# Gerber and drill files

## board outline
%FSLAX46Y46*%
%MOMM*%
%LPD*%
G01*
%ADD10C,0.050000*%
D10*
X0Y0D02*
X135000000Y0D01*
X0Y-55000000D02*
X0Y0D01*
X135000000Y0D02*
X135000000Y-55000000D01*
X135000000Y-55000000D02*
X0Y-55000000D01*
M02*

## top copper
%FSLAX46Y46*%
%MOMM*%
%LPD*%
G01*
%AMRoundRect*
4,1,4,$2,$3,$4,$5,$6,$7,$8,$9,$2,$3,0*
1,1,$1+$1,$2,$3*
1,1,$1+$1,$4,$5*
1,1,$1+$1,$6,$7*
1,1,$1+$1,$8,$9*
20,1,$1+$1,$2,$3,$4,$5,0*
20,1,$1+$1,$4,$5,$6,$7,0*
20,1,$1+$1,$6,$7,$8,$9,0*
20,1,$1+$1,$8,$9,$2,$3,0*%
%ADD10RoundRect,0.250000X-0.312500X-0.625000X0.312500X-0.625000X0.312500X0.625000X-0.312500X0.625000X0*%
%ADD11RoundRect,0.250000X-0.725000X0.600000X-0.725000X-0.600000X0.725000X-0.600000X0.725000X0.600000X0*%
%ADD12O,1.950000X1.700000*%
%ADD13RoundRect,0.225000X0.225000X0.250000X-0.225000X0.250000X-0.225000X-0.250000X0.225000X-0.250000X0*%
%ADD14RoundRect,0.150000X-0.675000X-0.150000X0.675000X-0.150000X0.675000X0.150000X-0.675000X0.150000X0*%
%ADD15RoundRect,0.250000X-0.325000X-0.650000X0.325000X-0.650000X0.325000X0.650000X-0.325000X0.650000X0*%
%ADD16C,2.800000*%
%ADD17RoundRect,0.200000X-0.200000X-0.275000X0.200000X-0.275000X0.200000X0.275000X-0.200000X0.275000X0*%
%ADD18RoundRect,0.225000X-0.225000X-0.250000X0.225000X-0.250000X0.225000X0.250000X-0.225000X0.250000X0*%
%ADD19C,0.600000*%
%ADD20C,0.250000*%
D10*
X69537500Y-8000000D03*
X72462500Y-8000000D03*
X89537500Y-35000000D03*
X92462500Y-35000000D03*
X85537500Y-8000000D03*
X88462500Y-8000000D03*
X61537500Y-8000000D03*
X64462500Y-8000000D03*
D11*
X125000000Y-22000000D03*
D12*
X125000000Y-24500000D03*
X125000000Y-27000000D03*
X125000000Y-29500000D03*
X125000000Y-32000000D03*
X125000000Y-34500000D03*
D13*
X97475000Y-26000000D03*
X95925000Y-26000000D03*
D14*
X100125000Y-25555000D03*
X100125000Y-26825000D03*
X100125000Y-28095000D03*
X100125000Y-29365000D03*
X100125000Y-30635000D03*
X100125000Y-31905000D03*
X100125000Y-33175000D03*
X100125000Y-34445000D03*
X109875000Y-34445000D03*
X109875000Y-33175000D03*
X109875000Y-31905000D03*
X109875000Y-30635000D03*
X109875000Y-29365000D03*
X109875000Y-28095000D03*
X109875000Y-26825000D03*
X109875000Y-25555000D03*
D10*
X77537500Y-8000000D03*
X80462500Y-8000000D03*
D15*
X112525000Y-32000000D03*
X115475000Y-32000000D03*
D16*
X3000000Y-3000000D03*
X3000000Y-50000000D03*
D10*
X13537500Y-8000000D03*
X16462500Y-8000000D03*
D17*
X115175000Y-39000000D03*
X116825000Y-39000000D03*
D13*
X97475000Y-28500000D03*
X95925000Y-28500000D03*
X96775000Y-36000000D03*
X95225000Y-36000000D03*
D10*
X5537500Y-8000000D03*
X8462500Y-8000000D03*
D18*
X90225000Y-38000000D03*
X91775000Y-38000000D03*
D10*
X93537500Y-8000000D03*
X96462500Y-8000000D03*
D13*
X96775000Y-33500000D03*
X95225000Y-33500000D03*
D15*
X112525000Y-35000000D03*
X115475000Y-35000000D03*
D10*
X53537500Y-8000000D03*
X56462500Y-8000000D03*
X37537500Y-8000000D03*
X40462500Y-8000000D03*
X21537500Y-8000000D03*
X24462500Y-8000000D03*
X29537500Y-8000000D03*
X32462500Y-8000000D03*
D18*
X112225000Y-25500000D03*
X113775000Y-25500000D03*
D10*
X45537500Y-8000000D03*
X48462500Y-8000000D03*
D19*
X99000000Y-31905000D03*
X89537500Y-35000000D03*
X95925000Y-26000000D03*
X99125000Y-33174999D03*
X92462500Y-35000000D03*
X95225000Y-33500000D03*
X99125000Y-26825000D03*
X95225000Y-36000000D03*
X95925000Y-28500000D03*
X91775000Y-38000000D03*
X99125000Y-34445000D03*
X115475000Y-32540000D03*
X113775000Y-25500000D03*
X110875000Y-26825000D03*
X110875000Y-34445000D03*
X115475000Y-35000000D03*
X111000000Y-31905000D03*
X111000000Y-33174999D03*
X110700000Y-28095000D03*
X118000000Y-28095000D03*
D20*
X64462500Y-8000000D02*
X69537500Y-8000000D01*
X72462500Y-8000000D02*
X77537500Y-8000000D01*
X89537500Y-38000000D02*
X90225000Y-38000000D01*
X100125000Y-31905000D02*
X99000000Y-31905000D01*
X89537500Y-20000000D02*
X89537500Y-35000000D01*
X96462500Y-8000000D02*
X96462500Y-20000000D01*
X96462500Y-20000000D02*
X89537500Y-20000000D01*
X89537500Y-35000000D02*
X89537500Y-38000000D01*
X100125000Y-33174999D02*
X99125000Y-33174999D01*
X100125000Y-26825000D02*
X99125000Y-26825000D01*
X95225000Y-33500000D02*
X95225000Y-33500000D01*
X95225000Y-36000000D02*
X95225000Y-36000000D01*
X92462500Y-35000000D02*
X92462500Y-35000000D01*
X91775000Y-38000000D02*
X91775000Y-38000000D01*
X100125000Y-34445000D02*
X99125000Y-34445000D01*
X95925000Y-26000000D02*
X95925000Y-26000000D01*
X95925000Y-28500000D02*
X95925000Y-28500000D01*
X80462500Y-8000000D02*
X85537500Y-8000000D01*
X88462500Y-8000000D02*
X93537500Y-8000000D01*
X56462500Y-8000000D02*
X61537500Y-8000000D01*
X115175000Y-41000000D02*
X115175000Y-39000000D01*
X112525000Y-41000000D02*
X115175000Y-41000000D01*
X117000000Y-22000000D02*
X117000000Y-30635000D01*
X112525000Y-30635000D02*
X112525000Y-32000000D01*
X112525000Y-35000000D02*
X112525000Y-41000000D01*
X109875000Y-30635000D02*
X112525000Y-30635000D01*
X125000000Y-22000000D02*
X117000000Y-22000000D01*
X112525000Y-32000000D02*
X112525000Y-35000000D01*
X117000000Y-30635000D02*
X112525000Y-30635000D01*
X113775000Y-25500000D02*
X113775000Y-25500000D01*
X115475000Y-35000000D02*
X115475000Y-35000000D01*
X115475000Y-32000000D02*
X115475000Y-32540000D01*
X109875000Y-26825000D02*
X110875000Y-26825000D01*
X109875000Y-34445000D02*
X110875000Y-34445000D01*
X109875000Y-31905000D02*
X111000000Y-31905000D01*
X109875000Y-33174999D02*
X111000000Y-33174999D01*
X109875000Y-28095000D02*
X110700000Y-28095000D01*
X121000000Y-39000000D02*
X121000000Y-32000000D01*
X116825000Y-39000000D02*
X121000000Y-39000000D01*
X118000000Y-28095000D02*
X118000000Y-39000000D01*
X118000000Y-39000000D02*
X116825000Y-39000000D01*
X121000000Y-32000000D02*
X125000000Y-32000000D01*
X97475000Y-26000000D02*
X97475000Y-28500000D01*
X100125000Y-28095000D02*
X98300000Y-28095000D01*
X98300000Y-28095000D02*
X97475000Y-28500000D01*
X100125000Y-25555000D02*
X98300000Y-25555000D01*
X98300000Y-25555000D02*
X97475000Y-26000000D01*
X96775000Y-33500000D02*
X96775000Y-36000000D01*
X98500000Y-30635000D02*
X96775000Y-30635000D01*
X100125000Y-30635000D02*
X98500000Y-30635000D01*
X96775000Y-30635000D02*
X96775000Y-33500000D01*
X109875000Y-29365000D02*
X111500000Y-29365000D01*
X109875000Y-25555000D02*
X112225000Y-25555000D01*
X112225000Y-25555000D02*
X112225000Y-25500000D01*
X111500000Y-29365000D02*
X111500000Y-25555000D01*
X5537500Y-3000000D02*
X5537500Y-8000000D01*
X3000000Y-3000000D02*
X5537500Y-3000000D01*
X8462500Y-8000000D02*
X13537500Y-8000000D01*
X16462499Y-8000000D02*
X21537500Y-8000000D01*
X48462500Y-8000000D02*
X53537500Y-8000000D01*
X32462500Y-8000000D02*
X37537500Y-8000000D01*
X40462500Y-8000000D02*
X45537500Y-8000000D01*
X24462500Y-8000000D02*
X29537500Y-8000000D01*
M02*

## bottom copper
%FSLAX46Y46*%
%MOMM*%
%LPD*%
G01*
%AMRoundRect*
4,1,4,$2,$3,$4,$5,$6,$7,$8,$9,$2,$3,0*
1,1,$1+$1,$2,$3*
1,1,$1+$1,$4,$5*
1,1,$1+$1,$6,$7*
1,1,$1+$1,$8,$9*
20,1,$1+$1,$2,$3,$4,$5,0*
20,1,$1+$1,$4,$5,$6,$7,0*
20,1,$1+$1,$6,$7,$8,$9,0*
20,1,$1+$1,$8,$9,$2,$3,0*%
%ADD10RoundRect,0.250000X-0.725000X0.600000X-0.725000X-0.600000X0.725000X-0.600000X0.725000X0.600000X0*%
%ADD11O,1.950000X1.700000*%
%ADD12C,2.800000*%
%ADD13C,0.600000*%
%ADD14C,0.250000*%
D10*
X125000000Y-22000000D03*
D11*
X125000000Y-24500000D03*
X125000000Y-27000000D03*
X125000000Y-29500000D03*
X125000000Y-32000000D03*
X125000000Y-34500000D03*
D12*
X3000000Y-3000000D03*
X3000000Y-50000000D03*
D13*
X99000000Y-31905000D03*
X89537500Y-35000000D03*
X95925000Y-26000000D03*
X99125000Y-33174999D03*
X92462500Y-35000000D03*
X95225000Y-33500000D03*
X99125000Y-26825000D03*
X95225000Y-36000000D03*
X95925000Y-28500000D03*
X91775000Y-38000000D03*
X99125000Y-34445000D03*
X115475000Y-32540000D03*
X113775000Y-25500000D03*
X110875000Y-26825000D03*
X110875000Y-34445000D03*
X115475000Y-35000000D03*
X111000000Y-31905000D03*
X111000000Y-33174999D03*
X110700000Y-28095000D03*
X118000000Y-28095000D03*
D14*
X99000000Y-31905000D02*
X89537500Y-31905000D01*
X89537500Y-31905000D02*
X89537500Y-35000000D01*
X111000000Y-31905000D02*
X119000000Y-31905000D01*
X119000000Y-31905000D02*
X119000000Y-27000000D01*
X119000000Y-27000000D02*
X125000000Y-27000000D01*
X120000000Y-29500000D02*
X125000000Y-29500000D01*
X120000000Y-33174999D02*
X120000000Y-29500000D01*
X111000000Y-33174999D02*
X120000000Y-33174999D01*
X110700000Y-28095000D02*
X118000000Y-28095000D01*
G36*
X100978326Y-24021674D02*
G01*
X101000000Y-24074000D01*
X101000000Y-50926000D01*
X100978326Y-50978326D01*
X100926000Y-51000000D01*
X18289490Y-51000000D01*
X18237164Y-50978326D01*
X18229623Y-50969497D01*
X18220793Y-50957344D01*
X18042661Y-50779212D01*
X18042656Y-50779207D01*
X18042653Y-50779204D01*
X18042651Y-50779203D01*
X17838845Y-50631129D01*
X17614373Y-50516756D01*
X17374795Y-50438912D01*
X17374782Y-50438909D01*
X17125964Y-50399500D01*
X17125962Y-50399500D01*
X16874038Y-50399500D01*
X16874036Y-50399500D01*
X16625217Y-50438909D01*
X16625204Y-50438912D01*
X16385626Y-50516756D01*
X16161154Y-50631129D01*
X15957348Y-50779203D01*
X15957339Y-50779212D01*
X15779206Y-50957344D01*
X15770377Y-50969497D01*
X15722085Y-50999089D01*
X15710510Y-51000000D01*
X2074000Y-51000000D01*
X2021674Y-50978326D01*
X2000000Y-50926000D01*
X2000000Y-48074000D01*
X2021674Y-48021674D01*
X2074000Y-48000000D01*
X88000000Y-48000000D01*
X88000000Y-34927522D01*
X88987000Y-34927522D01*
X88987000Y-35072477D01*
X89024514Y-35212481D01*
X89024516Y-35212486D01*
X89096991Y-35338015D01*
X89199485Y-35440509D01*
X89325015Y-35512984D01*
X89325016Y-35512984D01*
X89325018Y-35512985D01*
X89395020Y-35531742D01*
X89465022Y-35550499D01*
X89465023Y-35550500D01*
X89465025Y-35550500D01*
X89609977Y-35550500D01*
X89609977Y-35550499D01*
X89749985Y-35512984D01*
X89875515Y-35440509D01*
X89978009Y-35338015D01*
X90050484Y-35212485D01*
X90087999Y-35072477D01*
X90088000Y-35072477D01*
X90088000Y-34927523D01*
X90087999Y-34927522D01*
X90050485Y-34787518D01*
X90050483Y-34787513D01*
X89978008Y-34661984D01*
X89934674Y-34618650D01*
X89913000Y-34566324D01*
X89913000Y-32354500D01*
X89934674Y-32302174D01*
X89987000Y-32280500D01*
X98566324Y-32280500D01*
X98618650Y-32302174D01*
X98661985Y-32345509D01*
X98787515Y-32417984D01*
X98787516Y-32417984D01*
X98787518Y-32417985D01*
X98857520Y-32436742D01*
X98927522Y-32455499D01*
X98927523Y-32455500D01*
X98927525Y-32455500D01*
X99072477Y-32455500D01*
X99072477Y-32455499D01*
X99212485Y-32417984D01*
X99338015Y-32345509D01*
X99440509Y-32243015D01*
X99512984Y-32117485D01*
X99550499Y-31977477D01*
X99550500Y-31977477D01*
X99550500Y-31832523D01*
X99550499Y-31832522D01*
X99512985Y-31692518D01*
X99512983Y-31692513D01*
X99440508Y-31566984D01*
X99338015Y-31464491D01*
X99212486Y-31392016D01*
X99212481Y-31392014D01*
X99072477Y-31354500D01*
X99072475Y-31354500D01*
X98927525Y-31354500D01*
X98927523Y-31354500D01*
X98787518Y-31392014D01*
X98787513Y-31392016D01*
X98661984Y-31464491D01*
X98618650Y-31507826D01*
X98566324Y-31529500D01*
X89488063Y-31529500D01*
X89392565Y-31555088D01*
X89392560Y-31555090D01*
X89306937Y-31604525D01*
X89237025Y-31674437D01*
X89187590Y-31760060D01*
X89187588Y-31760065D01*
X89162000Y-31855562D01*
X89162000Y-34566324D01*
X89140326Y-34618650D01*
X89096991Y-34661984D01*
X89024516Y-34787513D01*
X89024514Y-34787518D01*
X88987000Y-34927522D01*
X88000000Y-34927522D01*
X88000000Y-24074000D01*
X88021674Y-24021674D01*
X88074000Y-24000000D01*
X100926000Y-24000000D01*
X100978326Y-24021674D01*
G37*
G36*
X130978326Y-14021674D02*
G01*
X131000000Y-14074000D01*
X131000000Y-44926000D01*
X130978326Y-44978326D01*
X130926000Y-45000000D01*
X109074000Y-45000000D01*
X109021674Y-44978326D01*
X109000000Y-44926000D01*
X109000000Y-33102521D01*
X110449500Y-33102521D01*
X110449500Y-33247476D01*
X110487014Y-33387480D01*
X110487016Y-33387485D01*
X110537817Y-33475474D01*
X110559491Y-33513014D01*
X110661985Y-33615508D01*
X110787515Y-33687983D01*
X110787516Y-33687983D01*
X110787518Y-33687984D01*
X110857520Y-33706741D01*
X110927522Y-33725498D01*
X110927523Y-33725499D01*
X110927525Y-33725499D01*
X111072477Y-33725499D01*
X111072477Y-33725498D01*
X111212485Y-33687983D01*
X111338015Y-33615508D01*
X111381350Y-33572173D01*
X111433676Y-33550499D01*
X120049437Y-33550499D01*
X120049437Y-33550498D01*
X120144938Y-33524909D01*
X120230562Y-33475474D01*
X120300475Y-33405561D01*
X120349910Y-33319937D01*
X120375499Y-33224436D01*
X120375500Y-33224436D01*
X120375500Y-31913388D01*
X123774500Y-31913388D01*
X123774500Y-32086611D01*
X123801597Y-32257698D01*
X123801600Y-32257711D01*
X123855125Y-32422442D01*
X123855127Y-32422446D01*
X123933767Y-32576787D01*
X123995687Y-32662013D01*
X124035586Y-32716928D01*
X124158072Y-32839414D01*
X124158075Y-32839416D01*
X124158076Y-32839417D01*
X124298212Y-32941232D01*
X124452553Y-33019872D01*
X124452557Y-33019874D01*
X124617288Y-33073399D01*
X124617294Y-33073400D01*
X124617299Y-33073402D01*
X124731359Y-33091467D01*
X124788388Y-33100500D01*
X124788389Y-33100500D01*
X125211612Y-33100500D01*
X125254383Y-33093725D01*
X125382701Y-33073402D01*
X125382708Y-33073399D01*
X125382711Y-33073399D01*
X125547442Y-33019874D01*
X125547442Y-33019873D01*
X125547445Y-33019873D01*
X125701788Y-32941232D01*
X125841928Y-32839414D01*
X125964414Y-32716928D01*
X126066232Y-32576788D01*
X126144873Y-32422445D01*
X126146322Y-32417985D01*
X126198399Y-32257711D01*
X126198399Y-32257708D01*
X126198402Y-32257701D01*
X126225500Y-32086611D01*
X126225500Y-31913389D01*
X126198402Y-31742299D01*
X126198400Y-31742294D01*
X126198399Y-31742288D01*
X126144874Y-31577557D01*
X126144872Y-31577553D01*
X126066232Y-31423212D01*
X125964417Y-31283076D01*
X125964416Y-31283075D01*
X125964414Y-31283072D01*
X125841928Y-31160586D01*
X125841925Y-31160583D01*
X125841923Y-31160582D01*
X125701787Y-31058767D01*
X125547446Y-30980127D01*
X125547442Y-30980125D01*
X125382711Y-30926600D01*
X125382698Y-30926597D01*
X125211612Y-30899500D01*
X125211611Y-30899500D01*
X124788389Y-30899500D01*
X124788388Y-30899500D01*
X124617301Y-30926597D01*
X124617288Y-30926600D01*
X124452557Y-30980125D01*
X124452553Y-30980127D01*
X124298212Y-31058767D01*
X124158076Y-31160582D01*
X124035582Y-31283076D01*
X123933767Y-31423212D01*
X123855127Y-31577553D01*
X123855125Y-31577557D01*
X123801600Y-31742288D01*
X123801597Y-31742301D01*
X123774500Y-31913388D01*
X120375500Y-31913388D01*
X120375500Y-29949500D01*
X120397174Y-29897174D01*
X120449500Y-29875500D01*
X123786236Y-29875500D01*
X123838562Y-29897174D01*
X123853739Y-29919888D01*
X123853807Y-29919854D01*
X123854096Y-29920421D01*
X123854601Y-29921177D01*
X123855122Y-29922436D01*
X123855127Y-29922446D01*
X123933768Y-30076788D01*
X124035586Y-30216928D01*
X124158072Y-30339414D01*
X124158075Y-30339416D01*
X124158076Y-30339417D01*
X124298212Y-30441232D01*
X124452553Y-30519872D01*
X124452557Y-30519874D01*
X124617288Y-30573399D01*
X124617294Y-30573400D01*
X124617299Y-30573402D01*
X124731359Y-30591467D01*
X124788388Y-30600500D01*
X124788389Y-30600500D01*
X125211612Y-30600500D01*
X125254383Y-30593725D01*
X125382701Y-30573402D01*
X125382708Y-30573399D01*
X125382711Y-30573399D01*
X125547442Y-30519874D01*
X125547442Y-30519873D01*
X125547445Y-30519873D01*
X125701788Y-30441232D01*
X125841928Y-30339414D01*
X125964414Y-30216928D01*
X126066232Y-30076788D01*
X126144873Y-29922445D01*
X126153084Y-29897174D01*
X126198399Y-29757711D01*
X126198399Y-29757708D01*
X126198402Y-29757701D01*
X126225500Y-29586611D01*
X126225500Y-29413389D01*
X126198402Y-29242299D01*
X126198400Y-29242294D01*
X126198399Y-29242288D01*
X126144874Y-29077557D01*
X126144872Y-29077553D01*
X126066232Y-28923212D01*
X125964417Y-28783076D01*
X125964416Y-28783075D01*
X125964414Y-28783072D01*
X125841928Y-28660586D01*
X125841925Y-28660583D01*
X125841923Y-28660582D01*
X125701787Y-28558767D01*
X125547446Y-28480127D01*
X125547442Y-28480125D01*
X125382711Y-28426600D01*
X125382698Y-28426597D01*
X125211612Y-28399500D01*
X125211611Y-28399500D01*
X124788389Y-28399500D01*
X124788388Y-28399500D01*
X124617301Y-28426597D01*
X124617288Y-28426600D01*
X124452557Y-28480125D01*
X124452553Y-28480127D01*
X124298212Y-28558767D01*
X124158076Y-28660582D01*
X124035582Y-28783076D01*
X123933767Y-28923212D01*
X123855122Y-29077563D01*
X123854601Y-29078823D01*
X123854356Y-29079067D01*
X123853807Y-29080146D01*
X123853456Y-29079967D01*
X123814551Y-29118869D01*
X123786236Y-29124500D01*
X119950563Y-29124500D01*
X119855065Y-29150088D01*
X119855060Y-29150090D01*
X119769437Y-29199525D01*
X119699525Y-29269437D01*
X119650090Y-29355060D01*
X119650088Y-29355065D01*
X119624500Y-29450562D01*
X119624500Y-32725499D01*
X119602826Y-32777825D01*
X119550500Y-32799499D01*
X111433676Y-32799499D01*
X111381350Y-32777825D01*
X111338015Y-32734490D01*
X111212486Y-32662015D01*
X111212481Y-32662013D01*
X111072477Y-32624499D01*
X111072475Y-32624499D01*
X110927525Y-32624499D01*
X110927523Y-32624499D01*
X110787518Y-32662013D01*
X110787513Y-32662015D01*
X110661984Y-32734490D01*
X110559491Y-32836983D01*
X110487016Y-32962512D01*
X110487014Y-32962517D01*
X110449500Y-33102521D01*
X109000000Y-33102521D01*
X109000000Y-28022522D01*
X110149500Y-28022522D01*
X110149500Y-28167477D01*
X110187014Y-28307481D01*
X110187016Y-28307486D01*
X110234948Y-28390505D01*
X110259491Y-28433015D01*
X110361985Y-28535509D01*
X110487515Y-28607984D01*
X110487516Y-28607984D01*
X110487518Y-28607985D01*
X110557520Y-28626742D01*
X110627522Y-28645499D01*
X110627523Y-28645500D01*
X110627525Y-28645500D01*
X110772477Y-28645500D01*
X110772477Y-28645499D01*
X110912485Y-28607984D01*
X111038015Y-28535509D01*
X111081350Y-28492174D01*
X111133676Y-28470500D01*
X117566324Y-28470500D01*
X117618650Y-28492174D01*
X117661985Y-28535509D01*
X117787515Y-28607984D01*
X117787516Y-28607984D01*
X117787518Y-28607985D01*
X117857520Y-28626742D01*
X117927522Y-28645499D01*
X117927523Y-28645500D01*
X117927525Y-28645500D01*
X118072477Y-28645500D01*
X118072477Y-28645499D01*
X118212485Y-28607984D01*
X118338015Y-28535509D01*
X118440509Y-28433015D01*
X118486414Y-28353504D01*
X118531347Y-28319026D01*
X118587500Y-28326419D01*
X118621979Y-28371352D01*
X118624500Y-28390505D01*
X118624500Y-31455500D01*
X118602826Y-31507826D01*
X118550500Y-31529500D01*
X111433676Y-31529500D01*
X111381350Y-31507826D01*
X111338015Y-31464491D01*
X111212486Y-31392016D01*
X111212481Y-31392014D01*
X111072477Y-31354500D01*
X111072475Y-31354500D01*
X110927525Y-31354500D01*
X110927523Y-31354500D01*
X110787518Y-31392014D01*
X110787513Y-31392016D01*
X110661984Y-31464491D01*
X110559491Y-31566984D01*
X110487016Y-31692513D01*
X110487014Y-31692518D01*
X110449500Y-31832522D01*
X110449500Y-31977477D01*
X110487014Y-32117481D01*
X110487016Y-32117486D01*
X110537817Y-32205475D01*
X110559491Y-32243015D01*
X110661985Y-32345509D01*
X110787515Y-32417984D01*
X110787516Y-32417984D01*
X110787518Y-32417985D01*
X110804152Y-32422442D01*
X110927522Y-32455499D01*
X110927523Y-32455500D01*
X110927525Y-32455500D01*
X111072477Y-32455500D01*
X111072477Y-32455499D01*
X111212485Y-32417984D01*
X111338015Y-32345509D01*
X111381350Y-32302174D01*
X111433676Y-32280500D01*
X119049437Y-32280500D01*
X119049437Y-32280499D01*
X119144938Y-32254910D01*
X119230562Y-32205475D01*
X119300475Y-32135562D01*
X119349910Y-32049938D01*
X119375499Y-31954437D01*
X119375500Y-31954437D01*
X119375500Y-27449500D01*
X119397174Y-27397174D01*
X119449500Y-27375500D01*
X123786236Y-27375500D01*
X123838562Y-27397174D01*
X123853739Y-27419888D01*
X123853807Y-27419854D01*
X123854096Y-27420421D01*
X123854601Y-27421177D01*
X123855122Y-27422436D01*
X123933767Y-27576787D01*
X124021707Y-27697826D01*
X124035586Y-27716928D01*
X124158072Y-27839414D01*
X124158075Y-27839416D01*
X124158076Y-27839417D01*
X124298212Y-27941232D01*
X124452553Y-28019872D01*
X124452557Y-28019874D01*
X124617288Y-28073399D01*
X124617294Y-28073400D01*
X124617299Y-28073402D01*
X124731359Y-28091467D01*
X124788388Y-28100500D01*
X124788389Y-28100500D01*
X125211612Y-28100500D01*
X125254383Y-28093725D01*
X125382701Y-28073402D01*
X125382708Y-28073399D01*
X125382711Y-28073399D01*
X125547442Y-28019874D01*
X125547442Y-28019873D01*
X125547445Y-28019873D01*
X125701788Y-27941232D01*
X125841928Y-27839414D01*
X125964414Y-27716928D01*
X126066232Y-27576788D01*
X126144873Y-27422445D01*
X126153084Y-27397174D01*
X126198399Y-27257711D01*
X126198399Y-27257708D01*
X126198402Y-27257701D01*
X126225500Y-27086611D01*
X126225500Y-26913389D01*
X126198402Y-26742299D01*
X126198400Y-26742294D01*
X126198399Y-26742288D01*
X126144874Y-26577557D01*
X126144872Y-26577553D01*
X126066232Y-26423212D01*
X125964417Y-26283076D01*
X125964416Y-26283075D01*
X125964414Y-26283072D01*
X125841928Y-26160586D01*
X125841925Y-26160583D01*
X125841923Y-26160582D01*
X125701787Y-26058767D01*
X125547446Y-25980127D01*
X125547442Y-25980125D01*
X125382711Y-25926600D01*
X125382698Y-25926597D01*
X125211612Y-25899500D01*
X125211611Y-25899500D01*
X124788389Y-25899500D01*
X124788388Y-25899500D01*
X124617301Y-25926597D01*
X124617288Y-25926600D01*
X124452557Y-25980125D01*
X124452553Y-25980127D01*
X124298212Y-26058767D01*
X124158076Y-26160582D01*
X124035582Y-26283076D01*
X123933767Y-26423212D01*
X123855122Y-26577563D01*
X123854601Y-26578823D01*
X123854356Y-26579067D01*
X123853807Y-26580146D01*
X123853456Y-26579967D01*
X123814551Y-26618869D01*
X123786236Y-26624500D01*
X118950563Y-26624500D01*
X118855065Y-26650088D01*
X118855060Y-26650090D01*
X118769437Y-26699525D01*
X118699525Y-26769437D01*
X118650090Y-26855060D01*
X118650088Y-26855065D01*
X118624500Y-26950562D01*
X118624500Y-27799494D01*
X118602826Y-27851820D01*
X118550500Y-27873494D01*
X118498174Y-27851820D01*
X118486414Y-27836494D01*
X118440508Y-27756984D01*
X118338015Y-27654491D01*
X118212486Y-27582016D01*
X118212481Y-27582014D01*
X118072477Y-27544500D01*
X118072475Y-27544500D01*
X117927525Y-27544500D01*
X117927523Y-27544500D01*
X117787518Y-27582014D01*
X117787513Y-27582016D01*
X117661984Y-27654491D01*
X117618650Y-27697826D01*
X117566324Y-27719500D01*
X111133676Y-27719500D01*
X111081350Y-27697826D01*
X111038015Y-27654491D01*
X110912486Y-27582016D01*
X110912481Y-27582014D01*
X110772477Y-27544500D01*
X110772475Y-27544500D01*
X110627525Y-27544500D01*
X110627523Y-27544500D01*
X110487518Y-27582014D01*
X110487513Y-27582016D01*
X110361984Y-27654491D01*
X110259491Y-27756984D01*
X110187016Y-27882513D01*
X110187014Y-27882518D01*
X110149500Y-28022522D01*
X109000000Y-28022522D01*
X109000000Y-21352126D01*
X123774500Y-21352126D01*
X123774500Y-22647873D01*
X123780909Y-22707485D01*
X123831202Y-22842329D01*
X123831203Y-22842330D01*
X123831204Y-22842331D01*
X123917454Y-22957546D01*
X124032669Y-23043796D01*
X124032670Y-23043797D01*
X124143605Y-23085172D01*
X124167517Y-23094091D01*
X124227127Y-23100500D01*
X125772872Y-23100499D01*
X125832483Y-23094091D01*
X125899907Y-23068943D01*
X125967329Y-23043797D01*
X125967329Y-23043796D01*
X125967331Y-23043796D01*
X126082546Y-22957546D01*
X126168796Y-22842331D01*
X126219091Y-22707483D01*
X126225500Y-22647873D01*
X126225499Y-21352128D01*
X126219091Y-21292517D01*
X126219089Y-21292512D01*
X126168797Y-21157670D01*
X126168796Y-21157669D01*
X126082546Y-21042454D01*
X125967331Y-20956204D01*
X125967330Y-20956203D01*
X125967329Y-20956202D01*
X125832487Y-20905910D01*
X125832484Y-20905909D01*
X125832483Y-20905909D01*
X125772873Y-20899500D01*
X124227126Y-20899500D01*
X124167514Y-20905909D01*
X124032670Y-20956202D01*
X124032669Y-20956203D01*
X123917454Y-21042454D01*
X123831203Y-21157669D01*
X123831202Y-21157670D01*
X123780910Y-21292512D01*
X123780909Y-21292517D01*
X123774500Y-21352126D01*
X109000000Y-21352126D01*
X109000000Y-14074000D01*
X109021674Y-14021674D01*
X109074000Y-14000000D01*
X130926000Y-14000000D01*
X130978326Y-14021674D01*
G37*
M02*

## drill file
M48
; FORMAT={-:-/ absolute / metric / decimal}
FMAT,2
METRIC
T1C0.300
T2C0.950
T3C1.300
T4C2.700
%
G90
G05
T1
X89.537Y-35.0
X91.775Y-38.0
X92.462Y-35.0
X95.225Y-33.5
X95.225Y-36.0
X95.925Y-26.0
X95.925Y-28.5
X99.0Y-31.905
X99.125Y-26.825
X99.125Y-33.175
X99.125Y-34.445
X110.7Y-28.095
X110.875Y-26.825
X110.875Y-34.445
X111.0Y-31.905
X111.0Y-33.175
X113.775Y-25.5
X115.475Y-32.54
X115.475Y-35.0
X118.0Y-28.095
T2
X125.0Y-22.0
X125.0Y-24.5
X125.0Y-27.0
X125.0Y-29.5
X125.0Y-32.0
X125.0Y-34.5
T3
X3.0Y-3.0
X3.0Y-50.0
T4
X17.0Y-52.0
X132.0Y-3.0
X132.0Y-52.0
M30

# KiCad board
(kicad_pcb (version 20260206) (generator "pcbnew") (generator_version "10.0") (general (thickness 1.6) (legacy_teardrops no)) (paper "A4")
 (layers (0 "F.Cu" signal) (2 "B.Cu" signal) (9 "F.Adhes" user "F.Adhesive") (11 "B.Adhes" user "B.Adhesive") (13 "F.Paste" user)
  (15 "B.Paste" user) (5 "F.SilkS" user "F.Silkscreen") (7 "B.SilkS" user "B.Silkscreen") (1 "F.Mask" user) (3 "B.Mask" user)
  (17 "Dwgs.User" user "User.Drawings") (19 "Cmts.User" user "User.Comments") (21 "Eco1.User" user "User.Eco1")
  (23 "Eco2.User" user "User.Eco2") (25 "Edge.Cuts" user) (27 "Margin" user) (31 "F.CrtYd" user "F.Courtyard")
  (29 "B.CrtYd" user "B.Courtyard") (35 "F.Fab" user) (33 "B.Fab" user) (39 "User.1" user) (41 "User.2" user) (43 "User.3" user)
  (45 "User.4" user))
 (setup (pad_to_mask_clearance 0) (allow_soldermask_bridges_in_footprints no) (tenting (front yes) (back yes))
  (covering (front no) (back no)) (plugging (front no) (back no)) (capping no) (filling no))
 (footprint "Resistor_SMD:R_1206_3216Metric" (layer "F.Cu") (at 71 8)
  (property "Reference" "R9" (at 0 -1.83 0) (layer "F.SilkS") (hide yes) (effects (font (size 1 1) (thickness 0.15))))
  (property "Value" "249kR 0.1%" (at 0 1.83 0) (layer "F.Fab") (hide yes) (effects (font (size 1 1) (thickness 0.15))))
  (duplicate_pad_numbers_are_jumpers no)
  (pad "1" smd roundrect (at -1.4625 0) (size 1.125 1.75) (layers "F.Cu" "F.Mask" "F.Paste") (roundrect_rratio 0.222222) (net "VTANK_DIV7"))
  (pad "2" smd roundrect (at 1.4625 0) (size 1.125 1.75) (layers "F.Cu" "F.Mask" "F.Paste") (roundrect_rratio 0.222222) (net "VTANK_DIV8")))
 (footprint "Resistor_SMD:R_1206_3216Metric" (layer "F.Cu") (at 91 35)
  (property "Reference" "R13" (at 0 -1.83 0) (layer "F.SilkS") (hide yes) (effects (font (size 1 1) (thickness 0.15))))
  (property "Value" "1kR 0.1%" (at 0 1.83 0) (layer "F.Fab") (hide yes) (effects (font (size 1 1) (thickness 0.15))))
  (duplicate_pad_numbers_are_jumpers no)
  (pad "1" smd roundrect (at -1.4625 0) (size 1.125 1.75) (layers "F.Cu" "F.Mask" "F.Paste") (roundrect_rratio 0.222222) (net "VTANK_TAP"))
  (pad "2" smd roundrect (at 1.4625 0) (size 1.125 1.75) (layers "F.Cu" "F.Mask" "F.Paste") (roundrect_rratio 0.222222) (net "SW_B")))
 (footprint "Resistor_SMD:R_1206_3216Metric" (layer "F.Cu") (at 87 8)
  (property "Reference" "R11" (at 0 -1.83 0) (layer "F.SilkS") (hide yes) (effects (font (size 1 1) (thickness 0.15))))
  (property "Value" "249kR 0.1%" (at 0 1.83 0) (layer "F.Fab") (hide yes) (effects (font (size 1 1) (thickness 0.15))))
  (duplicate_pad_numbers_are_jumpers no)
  (pad "1" smd roundrect (at -1.4625 0) (size 1.125 1.75) (layers "F.Cu" "F.Mask" "F.Paste") (roundrect_rratio 0.222222) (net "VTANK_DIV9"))
  (pad "2" smd roundrect (at 1.4625 0) (size 1.125 1.75) (layers "F.Cu" "F.Mask" "F.Paste") (roundrect_rratio 0.222222) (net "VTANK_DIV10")))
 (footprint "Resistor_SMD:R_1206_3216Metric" (layer "F.Cu") (at 63 8)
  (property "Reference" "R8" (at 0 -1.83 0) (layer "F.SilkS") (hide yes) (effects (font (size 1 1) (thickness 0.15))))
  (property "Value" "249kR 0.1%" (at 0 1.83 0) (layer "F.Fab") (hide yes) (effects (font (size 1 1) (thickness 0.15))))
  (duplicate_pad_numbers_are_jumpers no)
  (pad "1" smd roundrect (at -1.4625 0) (size 1.125 1.75) (layers "F.Cu" "F.Mask" "F.Paste") (roundrect_rratio 0.222222) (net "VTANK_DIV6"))
  (pad "2" smd roundrect (at 1.4625 0) (size 1.125 1.75) (layers "F.Cu" "F.Mask" "F.Paste") (roundrect_rratio 0.222222) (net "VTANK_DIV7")))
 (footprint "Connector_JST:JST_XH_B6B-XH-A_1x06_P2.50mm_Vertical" (layer "F.Cu") (at 125 22 -90)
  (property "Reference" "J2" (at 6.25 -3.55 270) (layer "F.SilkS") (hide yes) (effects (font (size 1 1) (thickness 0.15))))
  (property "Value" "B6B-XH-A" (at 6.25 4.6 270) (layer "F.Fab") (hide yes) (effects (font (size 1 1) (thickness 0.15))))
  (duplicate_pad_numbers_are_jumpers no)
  (pad "1" thru_hole roundrect (at 0 0 270) (size 1.7 1.95) (drill 0.95) (layers "*.Cu" "*.Mask") (remove_unused_layers no)
   (roundrect_rratio 0.147059) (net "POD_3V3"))
  (pad "2" thru_hole oval (at 2.5 0 270) (size 1.7 1.95) (drill 0.95) (layers "*.Cu" "*.Mask") (remove_unused_layers no) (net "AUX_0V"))
  (pad "3" thru_hole oval (at 5 0 270) (size 1.7 1.95) (drill 0.95) (layers "*.Cu" "*.Mask") (remove_unused_layers no) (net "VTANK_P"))
  (pad "4" thru_hole oval (at 7.5 0 270) (size 1.7 1.95) (drill 0.95) (layers "*.Cu" "*.Mask") (remove_unused_layers no) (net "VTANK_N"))
  (pad "5" thru_hole oval (at 10 0 270) (size 1.7 1.95) (drill 0.95) (layers "*.Cu" "*.Mask") (remove_unused_layers no) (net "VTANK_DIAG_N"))
  (pad "6" thru_hole oval (at 12.5 0 270) (size 1.7 1.95) (drill 0.95) (layers "*.Cu" "*.Mask") (remove_unused_layers no) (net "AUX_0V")))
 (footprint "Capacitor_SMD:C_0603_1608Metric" (layer "F.Cu") (at 96.7 26 180)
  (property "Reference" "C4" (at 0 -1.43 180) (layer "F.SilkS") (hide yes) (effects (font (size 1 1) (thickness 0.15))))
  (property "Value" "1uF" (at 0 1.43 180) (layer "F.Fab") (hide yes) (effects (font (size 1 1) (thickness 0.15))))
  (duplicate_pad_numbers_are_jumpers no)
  (pad "1" smd roundrect (at -0.775 0 180) (size 0.9 0.95) (layers "F.Cu" "F.Mask" "F.Paste") (roundrect_rratio 0.25) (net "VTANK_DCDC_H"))
  (pad "2" smd roundrect (at 0.775 0 180) (size 0.9 0.95) (layers "F.Cu" "F.Mask" "F.Paste") (roundrect_rratio 0.25) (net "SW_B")))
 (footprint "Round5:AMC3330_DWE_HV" (layer "F.Cu") (at 105 30)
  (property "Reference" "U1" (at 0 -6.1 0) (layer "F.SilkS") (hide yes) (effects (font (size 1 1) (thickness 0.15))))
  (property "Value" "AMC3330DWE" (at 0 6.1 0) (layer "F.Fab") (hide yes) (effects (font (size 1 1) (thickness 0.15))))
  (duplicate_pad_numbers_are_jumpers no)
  (pad "1" smd roundrect (at -4.875 -4.445) (size 1.65 0.6) (layers "F.Cu" "F.Mask" "F.Paste") (roundrect_rratio 0.25) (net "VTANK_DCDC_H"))
  (pad "2" smd roundrect (at -4.875 -3.175) (size 1.65 0.6) (layers "F.Cu" "F.Mask" "F.Paste") (roundrect_rratio 0.25) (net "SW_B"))
  (pad "3" smd roundrect (at -4.875 -1.905) (size 1.65 0.6) (layers "F.Cu" "F.Mask" "F.Paste") (roundrect_rratio 0.25) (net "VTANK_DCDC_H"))
  (pad "4" smd roundrect (at -4.875 -0.635) (size 1.65 0.6) (layers "F.Cu" "F.Mask" "F.Paste") (roundrect_rratio 0.25)
   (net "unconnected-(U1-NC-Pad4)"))
  (pad "5" smd roundrect (at -4.875 0.635) (size 1.65 0.6) (layers "F.Cu" "F.Mask" "F.Paste") (roundrect_rratio 0.25) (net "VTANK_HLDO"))
  (pad "6" smd roundrect (at -4.875 1.905) (size 1.65 0.6) (layers "F.Cu" "F.Mask" "F.Paste") (roundrect_rratio 0.25) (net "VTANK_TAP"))
  (pad "7" smd roundrect (at -4.875 3.175) (size 1.65 0.6) (layers "F.Cu" "F.Mask" "F.Paste") (roundrect_rratio 0.25) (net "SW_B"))
  (pad "8" smd roundrect (at -4.875 4.445) (size 1.65 0.6) (layers "F.Cu" "F.Mask" "F.Paste") (roundrect_rratio 0.25) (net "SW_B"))
  (pad "9" smd roundrect (at 4.875 4.445) (size 1.65 0.6) (layers "F.Cu" "F.Mask" "F.Paste") (roundrect_rratio 0.25) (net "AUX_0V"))
  (pad "10" smd roundrect (at 4.875 3.175) (size 1.65 0.6) (layers "F.Cu" "F.Mask" "F.Paste") (roundrect_rratio 0.25) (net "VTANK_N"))
  (pad "11" smd roundrect (at 4.875 1.905) (size 1.65 0.6) (layers "F.Cu" "F.Mask" "F.Paste") (roundrect_rratio 0.25) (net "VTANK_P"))
  (pad "12" smd roundrect (at 4.875 0.635) (size 1.65 0.6) (layers "F.Cu" "F.Mask" "F.Paste") (roundrect_rratio 0.25) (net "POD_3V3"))
  (pad "13" smd roundrect (at 4.875 -0.635) (size 1.65 0.6) (layers "F.Cu" "F.Mask" "F.Paste") (roundrect_rratio 0.25) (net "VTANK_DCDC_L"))
  (pad "14" smd roundrect (at 4.875 -1.905) (size 1.65 0.6) (layers "F.Cu" "F.Mask" "F.Paste") (roundrect_rratio 0.25) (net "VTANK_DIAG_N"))
  (pad "15" smd roundrect (at 4.875 -3.175) (size 1.65 0.6) (layers "F.Cu" "F.Mask" "F.Paste") (roundrect_rratio 0.25) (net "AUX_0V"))
  (pad "16" smd roundrect (at 4.875 -4.445) (size 1.65 0.6) (layers "F.Cu" "F.Mask" "F.Paste") (roundrect_rratio 0.25) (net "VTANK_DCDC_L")))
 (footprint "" (layer "F.Cu") (at 132 52)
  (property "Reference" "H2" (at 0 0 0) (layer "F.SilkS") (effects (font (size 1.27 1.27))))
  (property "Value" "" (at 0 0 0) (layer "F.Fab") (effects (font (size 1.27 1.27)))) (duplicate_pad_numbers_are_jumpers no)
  (pad "" np_thru_hole circle (at 0 0) (size 2.7 2.7) (drill 2.7) (layers "*.Cu")))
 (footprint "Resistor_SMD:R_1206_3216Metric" (layer "F.Cu") (at 79 8)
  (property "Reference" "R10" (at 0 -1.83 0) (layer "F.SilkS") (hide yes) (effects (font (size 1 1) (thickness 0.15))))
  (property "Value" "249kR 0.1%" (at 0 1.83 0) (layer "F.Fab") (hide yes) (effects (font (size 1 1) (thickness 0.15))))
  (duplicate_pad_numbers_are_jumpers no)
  (pad "1" smd roundrect (at -1.4625 0) (size 1.125 1.75) (layers "F.Cu" "F.Mask" "F.Paste") (roundrect_rratio 0.222222) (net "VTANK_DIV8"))
  (pad "2" smd roundrect (at 1.4625 0) (size 1.125 1.75) (layers "F.Cu" "F.Mask" "F.Paste") (roundrect_rratio 0.222222) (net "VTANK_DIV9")))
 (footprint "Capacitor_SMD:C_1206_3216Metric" (layer "F.Cu") (at 114 32)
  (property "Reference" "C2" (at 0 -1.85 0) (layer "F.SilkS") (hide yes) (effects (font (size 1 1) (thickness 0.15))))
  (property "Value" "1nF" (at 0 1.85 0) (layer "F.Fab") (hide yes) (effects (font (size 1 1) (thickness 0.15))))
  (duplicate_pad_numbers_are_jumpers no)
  (pad "1" smd roundrect (at -1.475 0) (size 1.15 1.8) (layers "F.Cu" "F.Mask" "F.Paste") (roundrect_rratio 0.217391) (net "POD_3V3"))
  (pad "2" smd roundrect (at 1.475 0) (size 1.15 1.8) (layers "F.Cu" "F.Mask" "F.Paste") (roundrect_rratio 0.217391) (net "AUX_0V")))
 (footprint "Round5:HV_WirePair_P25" (layer "F.Cu") (at 3 3)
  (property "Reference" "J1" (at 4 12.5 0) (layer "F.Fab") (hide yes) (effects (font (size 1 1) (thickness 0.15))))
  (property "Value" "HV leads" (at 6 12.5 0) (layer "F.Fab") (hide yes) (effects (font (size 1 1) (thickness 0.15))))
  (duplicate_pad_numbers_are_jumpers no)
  (pad "1" thru_hole circle (at 0 0) (size 2.8 2.8) (drill 1.3) (layers "*.Cu" "*.Mask") (remove_unused_layers no) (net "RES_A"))
  (pad "2" thru_hole circle (at 0 47) (size 2.8 2.8) (drill 1.3) (layers "*.Cu" "*.Mask") (remove_unused_layers no) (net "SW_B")))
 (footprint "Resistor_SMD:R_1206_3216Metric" (layer "F.Cu") (at 15 8)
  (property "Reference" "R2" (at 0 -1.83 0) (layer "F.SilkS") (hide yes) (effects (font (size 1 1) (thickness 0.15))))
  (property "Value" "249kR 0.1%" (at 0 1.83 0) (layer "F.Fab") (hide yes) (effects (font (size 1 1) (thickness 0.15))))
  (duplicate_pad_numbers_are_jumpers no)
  (pad "1" smd roundrect (at -1.4625 0) (size 1.125 1.75) (layers "F.Cu" "F.Mask" "F.Paste") (roundrect_rratio 0.222222) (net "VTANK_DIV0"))
  (pad "2" smd roundrect (at 1.4625 0) (size 1.125 1.75) (layers "F.Cu" "F.Mask" "F.Paste") (roundrect_rratio 0.222222) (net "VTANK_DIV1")))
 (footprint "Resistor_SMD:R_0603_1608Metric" (layer "F.Cu") (at 116 39)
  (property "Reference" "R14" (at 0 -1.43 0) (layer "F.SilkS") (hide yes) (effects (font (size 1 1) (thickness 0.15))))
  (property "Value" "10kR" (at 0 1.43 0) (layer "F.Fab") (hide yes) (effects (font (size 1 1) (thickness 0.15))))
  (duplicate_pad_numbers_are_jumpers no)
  (pad "1" smd roundrect (at -0.825 0) (size 0.8 0.95) (layers "F.Cu" "F.Mask" "F.Paste") (roundrect_rratio 0.25) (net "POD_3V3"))
  (pad "2" smd roundrect (at 0.825 0) (size 0.8 0.95) (layers "F.Cu" "F.Mask" "F.Paste") (roundrect_rratio 0.25) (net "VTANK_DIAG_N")))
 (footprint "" (layer "F.Cu") (at 17 52)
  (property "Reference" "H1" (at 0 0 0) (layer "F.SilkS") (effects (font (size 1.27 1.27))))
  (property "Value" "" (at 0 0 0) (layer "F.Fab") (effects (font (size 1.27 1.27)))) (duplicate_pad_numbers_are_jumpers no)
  (pad "" np_thru_hole circle (at 0 0) (size 2.7 2.7) (drill 2.7) (layers "*.Cu")))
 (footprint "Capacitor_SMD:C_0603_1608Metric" (layer "F.Cu") (at 96.7 28.5 180)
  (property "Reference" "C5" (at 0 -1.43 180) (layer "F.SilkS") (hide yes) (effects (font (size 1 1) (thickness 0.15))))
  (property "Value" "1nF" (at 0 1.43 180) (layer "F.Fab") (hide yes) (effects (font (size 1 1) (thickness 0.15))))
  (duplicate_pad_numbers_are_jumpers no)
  (pad "1" smd roundrect (at -0.775 0 180) (size 0.9 0.95) (layers "F.Cu" "F.Mask" "F.Paste") (roundrect_rratio 0.25) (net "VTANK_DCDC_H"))
  (pad "2" smd roundrect (at 0.775 0 180) (size 0.9 0.95) (layers "F.Cu" "F.Mask" "F.Paste") (roundrect_rratio 0.25) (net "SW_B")))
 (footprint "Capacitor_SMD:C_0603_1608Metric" (layer "F.Cu") (at 96 36 180)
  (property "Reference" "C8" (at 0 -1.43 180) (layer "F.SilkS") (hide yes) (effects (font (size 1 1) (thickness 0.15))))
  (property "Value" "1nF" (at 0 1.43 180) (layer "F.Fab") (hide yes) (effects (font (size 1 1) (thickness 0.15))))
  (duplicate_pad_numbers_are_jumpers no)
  (pad "1" smd roundrect (at -0.775 0 180) (size 0.9 0.95) (layers "F.Cu" "F.Mask" "F.Paste") (roundrect_rratio 0.25) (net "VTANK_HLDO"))
  (pad "2" smd roundrect (at 0.775 0 180) (size 0.9 0.95) (layers "F.Cu" "F.Mask" "F.Paste") (roundrect_rratio 0.25) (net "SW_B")))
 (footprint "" (layer "F.Cu") (at 132 3)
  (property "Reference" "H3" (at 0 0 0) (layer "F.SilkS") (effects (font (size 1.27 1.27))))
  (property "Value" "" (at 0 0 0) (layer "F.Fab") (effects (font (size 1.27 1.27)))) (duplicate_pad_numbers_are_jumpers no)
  (pad "" np_thru_hole circle (at 0 0) (size 2.7 2.7) (drill 2.7) (layers "*.Cu")))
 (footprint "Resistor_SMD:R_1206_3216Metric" (layer "F.Cu") (at 7 8)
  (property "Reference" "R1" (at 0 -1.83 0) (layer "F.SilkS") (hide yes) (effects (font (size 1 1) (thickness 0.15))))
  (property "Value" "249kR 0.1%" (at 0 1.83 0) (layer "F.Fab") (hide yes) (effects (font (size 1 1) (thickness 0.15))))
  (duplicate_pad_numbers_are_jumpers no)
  (pad "1" smd roundrect (at -1.4625 0) (size 1.125 1.75) (layers "F.Cu" "F.Mask" "F.Paste") (roundrect_rratio 0.222222) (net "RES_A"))
  (pad "2" smd roundrect (at 1.4625 0) (size 1.125 1.75) (layers "F.Cu" "F.Mask" "F.Paste") (roundrect_rratio 0.222222) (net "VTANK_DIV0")))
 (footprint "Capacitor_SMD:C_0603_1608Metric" (layer "F.Cu") (at 91 38)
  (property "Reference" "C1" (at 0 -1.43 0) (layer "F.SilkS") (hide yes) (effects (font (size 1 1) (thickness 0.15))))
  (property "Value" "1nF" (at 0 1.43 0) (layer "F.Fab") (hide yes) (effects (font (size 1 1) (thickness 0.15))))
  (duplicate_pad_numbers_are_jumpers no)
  (pad "1" smd roundrect (at -0.775 0) (size 0.9 0.95) (layers "F.Cu" "F.Mask" "F.Paste") (roundrect_rratio 0.25) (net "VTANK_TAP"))
  (pad "2" smd roundrect (at 0.775 0) (size 0.9 0.95) (layers "F.Cu" "F.Mask" "F.Paste") (roundrect_rratio 0.25) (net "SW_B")))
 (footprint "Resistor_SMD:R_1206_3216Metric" (layer "F.Cu") (at 95 8)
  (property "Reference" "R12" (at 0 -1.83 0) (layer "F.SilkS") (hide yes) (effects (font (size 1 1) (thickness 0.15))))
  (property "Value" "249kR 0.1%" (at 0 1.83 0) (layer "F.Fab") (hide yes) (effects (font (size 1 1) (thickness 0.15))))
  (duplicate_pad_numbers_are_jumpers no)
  (pad "1" smd roundrect (at -1.4625 0) (size 1.125 1.75) (layers "F.Cu" "F.Mask" "F.Paste") (roundrect_rratio 0.222222) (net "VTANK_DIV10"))
  (pad "2" smd roundrect (at 1.4625 0) (size 1.125 1.75) (layers "F.Cu" "F.Mask" "F.Paste") (roundrect_rratio 0.222222) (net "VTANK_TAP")))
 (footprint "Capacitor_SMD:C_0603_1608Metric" (layer "F.Cu") (at 96 33.5 180)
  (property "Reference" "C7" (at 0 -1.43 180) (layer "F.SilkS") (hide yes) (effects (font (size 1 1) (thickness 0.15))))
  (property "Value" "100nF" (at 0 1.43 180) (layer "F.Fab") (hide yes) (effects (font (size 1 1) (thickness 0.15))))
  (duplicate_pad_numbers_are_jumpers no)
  (pad "1" smd roundrect (at -0.775 0 180) (size 0.9 0.95) (layers "F.Cu" "F.Mask" "F.Paste") (roundrect_rratio 0.25) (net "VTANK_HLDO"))
  (pad "2" smd roundrect (at 0.775 0 180) (size 0.9 0.95) (layers "F.Cu" "F.Mask" "F.Paste") (roundrect_rratio 0.25) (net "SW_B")))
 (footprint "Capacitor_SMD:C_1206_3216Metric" (layer "F.Cu") (at 114 35)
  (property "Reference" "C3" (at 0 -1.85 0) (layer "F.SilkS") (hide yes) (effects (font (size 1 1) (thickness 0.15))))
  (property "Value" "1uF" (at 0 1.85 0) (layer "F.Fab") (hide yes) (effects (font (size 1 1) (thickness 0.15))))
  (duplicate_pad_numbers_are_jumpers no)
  (pad "1" smd roundrect (at -1.475 0) (size 1.15 1.8) (layers "F.Cu" "F.Mask" "F.Paste") (roundrect_rratio 0.217391) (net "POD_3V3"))
  (pad "2" smd roundrect (at 1.475 0) (size 1.15 1.8) (layers "F.Cu" "F.Mask" "F.Paste") (roundrect_rratio 0.217391) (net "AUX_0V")))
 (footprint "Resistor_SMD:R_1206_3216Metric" (layer "F.Cu") (at 55 8)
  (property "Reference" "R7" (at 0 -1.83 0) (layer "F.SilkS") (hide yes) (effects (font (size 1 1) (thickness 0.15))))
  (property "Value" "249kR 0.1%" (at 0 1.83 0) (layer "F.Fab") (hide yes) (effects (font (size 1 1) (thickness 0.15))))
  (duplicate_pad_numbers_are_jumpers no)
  (pad "1" smd roundrect (at -1.4625 0) (size 1.125 1.75) (layers "F.Cu" "F.Mask" "F.Paste") (roundrect_rratio 0.222222) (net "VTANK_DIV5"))
  (pad "2" smd roundrect (at 1.4625 0) (size 1.125 1.75) (layers "F.Cu" "F.Mask" "F.Paste") (roundrect_rratio 0.222222) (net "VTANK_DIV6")))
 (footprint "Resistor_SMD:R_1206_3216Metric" (layer "F.Cu") (at 39 8)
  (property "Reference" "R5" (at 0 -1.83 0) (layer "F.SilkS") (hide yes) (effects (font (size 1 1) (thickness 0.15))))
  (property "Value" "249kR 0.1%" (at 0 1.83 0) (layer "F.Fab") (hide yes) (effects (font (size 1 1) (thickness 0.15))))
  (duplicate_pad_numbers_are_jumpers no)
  (pad "1" smd roundrect (at -1.4625 0) (size 1.125 1.75) (layers "F.Cu" "F.Mask" "F.Paste") (roundrect_rratio 0.222222) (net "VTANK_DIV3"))
  (pad "2" smd roundrect (at 1.4625 0) (size 1.125 1.75) (layers "F.Cu" "F.Mask" "F.Paste") (roundrect_rratio 0.222222) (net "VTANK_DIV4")))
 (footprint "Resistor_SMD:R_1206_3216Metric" (layer "F.Cu") (at 23 8)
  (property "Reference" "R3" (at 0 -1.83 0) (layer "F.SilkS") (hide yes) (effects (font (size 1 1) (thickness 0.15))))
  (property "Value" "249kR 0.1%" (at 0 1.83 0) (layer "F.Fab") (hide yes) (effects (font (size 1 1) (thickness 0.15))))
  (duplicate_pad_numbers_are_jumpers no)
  (pad "1" smd roundrect (at -1.4625 0) (size 1.125 1.75) (layers "F.Cu" "F.Mask" "F.Paste") (roundrect_rratio 0.222222) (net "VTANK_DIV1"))
  (pad "2" smd roundrect (at 1.4625 0) (size 1.125 1.75) (layers "F.Cu" "F.Mask" "F.Paste") (roundrect_rratio 0.222222) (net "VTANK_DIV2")))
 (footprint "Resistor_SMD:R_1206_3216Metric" (layer "F.Cu") (at 31 8)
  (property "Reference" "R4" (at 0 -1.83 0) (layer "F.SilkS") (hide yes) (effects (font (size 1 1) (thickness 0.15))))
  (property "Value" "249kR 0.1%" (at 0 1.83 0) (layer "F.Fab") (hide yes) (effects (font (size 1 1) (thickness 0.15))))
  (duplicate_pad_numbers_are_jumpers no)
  (pad "1" smd roundrect (at -1.4625 0) (size 1.125 1.75) (layers "F.Cu" "F.Mask" "F.Paste") (roundrect_rratio 0.222222) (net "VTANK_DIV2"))
  (pad "2" smd roundrect (at 1.4625 0) (size 1.125 1.75) (layers "F.Cu" "F.Mask" "F.Paste") (roundrect_rratio 0.222222) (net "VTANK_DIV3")))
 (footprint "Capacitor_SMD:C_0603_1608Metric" (layer "F.Cu") (at 113 25.5)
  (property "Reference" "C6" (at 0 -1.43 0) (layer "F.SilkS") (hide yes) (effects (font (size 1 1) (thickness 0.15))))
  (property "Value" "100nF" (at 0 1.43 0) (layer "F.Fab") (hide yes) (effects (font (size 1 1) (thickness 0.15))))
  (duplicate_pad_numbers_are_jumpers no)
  (pad "1" smd roundrect (at -0.775 0) (size 0.9 0.95) (layers "F.Cu" "F.Mask" "F.Paste") (roundrect_rratio 0.25) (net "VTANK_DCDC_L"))
  (pad "2" smd roundrect (at 0.775 0) (size 0.9 0.95) (layers "F.Cu" "F.Mask" "F.Paste") (roundrect_rratio 0.25) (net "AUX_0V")))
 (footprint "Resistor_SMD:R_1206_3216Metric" (layer "F.Cu") (at 47 8)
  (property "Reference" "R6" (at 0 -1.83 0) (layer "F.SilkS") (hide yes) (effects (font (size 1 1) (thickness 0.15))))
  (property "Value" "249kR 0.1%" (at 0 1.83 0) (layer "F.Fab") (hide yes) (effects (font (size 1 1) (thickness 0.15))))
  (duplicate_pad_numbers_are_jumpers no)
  (pad "1" smd roundrect (at -1.4625 0) (size 1.125 1.75) (layers "F.Cu" "F.Mask" "F.Paste") (roundrect_rratio 0.222222) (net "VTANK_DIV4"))
  (pad "2" smd roundrect (at 1.4625 0) (size 1.125 1.75) (layers "F.Cu" "F.Mask" "F.Paste") (roundrect_rratio 0.222222) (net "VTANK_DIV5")))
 (gr_line (start 0 0) (end 135 0) (stroke (width 0.05) (type default)) (layer "Edge.Cuts"))
 (gr_line (start 0 55) (end 0 0) (stroke (width 0.05) (type default)) (layer "Edge.Cuts"))
 (gr_line (start 135 0) (end 135 55) (stroke (width 0.05) (type default)) (layer "Edge.Cuts"))
 (gr_line (start 135 55) (end 0 55) (stroke (width 0.05) (type default)) (layer "Edge.Cuts"))
 (segment (start 64.4625 8) (end 69.5375 8) (width 0.25) (layer "F.Cu") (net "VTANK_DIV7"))
 (segment (start 72.4625 8) (end 77.5375 8) (width 0.25) (layer "F.Cu") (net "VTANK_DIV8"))
 (segment (start 89.5375 38) (end 90.225 38) (width 0.25) (layer "F.Cu") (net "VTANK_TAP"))
 (segment (start 100.125 31.905) (end 99 31.905) (width 0.25) (layer "F.Cu") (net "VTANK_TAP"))
 (segment (start 89.5375 20) (end 89.5375 35) (width 0.25) (layer "F.Cu") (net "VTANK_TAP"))
 (segment (start 96.4625 8) (end 96.4625 20) (width 0.25) (layer "F.Cu") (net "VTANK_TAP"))
 (segment (start 96.4625 20) (end 89.5375 20) (width 0.25) (layer "F.Cu") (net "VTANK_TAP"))
 (segment (start 89.5375 35) (end 89.5375 38) (width 0.25) (layer "F.Cu") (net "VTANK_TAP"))
 (via (at 99 31.905) (size 0.6) (drill 0.3) (layers "F.Cu" "B.Cu") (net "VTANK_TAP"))
 (via (at 89.5375 35) (size 0.6) (drill 0.3) (layers "F.Cu" "B.Cu") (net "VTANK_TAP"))
 (segment (start 99 31.905) (end 89.5375 31.905) (width 0.25) (layer "B.Cu") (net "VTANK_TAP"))
 (segment (start 89.5375 31.905) (end 89.5375 35) (width 0.25) (layer "B.Cu") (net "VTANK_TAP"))
 (segment (start 100.125 33.174999) (end 99.125 33.174999) (width 0.25) (layer "F.Cu") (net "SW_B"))
 (segment (start 100.125 26.825) (end 99.125 26.825) (width 0.25) (layer "F.Cu") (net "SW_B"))
 (segment (start 95.225 33.5) (end 95.225 33.5) (width 0.25) (layer "F.Cu") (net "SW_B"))
 (segment (start 95.225 36) (end 95.225 36) (width 0.25) (layer "F.Cu") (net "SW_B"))
 (segment (start 92.4625 35) (end 92.4625 35) (width 0.25) (layer "F.Cu") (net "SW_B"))
 (segment (start 91.775 38) (end 91.775 38) (width 0.25) (layer "F.Cu") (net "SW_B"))
 (segment (start 100.125 34.445) (end 99.125 34.445) (width 0.25) (layer "F.Cu") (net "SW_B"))
 (segment (start 95.925 26) (end 95.925 26) (width 0.25) (layer "F.Cu") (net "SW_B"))
 (segment (start 95.925 28.5) (end 95.925 28.5) (width 0.25) (layer "F.Cu") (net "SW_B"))
 (via (at 95.925 26) (size 0.6) (drill 0.3) (layers "F.Cu" "B.Cu") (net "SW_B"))
 (via (at 99.125 33.174999) (size 0.6) (drill 0.3) (layers "F.Cu" "B.Cu") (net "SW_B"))
 (via (at 92.4625 35) (size 0.6) (drill 0.3) (layers "F.Cu" "B.Cu") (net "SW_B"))
 (via (at 95.225 33.5) (size 0.6) (drill 0.3) (layers "F.Cu" "B.Cu") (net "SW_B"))
 (via (at 99.125 26.825) (size 0.6) (drill 0.3) (layers "F.Cu" "B.Cu") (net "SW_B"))
 (via (at 95.225 36) (size 0.6) (drill 0.3) (layers "F.Cu" "B.Cu") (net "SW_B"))
 (via (at 95.925 28.5) (size 0.6) (drill 0.3) (layers "F.Cu" "B.Cu") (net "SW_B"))
 (via (at 91.775 38) (size 0.6) (drill 0.3) (layers "F.Cu" "B.Cu") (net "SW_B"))
 (via (at 99.125 34.445) (size 0.6) (drill 0.3) (layers "F.Cu" "B.Cu") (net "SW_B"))
 (segment (start 80.4625 8) (end 85.5375 8) (width 0.25) (layer "F.Cu") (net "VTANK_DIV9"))
 (segment (start 88.4625 8) (end 93.5375 8) (width 0.25) (layer "F.Cu") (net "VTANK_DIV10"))
 (segment (start 56.4625 8) (end 61.5375 8) (width 0.25) (layer "F.Cu") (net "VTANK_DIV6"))
 (segment (start 115.175 41) (end 115.175 39) (width 0.25) (layer "F.Cu") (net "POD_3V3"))
 (segment (start 112.525 41) (end 115.175 41) (width 0.25) (layer "F.Cu") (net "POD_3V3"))
 (segment (start 117 22) (end 117 30.635) (width 0.25) (layer "F.Cu") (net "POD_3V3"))
 (segment (start 112.525 30.635) (end 112.525 32) (width 0.25) (layer "F.Cu") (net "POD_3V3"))
 (segment (start 112.525 35) (end 112.525 41) (width 0.25) (layer "F.Cu") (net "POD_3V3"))
 (segment (start 109.875 30.635) (end 112.525 30.635) (width 0.25) (layer "F.Cu") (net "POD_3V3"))
 (segment (start 125 22) (end 117 22) (width 0.25) (layer "F.Cu") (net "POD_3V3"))
 (segment (start 112.525 32) (end 112.525 35) (width 0.25) (layer "F.Cu") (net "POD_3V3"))
 (segment (start 117 30.635) (end 112.525 30.635) (width 0.25) (layer "F.Cu") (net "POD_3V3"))
 (segment (start 113.775 25.5) (end 113.775 25.5) (width 0.25) (layer "F.Cu") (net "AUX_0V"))
 (segment (start 115.475 35) (end 115.475 35) (width 0.25) (layer "F.Cu") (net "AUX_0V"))
 (segment (start 115.475 32) (end 115.475 32.54) (width 0.25) (layer "F.Cu") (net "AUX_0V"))
 (segment (start 109.875 26.825) (end 110.875 26.825) (width 0.25) (layer "F.Cu") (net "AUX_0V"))
 (segment (start 109.875 34.445) (end 110.875 34.445) (width 0.25) (layer "F.Cu") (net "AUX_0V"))
 (via (at 115.475 32.54) (size 0.6) (drill 0.3) (layers "F.Cu" "B.Cu") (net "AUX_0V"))
 (via (at 113.775 25.5) (size 0.6) (drill 0.3) (layers "F.Cu" "B.Cu") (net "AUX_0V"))
 (via (at 110.875 26.825) (size 0.6) (drill 0.3) (layers "F.Cu" "B.Cu") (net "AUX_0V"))
 (via (at 110.875 34.445) (size 0.6) (drill 0.3) (layers "F.Cu" "B.Cu") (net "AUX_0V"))
 (via (at 115.475 35) (size 0.6) (drill 0.3) (layers "F.Cu" "B.Cu") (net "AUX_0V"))
 (segment (start 109.875 31.905) (end 111 31.905) (width 0.25) (layer "F.Cu") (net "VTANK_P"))
 (via (at 111 31.905) (size 0.6) (drill 0.3) (layers "F.Cu" "B.Cu") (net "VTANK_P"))
 (segment (start 111 31.905) (end 119 31.905) (width 0.25) (layer "B.Cu") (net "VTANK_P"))
 (segment (start 119 31.905) (end 119 27) (width 0.25) (layer "B.Cu") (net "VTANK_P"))
 (segment (start 119 27) (end 125 27) (width 0.25) (layer "B.Cu") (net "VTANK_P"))
 (segment (start 109.875 33.174999) (end 111 33.174999) (width 0.25) (layer "F.Cu") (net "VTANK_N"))
 (via (at 111 33.174999) (size 0.6) (drill 0.3) (layers "F.Cu" "B.Cu") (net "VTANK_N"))
 (segment (start 120 29.5) (end 125 29.5) (width 0.25) (layer "B.Cu") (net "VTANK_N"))
 (segment (start 120 33.174999) (end 120 29.5) (width 0.25) (layer "B.Cu") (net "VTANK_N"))
 (segment (start 111 33.174999) (end 120 33.174999) (width 0.25) (layer "B.Cu") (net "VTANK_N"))
 (segment (start 109.875 28.095) (end 110.7 28.095) (width 0.25) (layer "F.Cu") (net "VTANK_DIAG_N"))
 (segment (start 121 39) (end 121 32) (width 0.25) (layer "F.Cu") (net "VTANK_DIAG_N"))
 (segment (start 116.825 39) (end 121 39) (width 0.25) (layer "F.Cu") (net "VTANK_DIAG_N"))
 (segment (start 118 28.095) (end 118 39) (width 0.25) (layer "F.Cu") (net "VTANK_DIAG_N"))
 (segment (start 118 39) (end 116.825 39) (width 0.25) (layer "F.Cu") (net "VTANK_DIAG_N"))
 (segment (start 121 32) (end 125 32) (width 0.25) (layer "F.Cu") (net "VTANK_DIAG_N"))
 (via (at 110.7 28.095) (size 0.6) (drill 0.3) (layers "F.Cu" "B.Cu") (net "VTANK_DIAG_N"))
 (via (at 118 28.095) (size 0.6) (drill 0.3) (layers "F.Cu" "B.Cu") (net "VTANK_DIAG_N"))
 (segment (start 110.7 28.095) (end 118 28.095) (width 0.25) (layer "B.Cu") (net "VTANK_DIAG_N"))
 (segment (start 97.475 26) (end 97.475 28.5) (width 0.25) (layer "F.Cu") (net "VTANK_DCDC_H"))
 (segment (start 100.125 28.095) (end 98.3 28.095) (width 0.25) (layer "F.Cu") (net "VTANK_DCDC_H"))
 (segment (start 98.3 28.095) (end 97.475 28.5) (width 0.25) (layer "F.Cu") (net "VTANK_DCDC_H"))
 (segment (start 100.125 25.555) (end 98.3 25.555) (width 0.25) (layer "F.Cu") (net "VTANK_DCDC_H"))
 (segment (start 98.3 25.555) (end 97.475 26) (width 0.25) (layer "F.Cu") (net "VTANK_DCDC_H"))
 (segment (start 96.775 33.5) (end 96.775 36) (width 0.25) (layer "F.Cu") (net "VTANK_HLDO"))
 (segment (start 98.5 30.635) (end 96.775 30.635) (width 0.25) (layer "F.Cu") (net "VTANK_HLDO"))
 (segment (start 100.125 30.635) (end 98.5 30.635) (width 0.25) (layer "F.Cu") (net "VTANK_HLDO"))
 (segment (start 96.775 30.635) (end 96.775 33.5) (width 0.25) (layer "F.Cu") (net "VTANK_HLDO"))
 (segment (start 109.875 29.365) (end 111.5 29.365) (width 0.25) (layer "F.Cu") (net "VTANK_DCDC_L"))
 (segment (start 109.875 25.555) (end 112.225 25.555) (width 0.25) (layer "F.Cu") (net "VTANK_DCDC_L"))
 (segment (start 112.225 25.555) (end 112.225 25.5) (width 0.25) (layer "F.Cu") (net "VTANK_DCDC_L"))
 (segment (start 111.5 29.365) (end 111.5 25.555) (width 0.25) (layer "F.Cu") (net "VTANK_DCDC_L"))
 (segment (start 5.5375 3) (end 5.5375 8) (width 0.25) (layer "F.Cu") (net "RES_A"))
 (segment (start 3 3) (end 5.5375 3) (width 0.25) (layer "F.Cu") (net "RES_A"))
 (segment (start 8.4625 8) (end 13.5375 8) (width 0.25) (layer "F.Cu") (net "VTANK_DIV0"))
 (segment (start 16.462499 8) (end 21.5375 8) (width 0.25) (layer "F.Cu") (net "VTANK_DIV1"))
 (segment (start 48.4625 8) (end 53.5375 8) (width 0.25) (layer "F.Cu") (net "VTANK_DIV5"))
 (segment (start 32.4625 8) (end 37.5375 8) (width 0.25) (layer "F.Cu") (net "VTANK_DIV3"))
 (segment (start 40.4625 8) (end 45.5375 8) (width 0.25) (layer "F.Cu") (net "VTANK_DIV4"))
 (segment (start 24.4625 8) (end 29.5375 8) (width 0.25) (layer "F.Cu") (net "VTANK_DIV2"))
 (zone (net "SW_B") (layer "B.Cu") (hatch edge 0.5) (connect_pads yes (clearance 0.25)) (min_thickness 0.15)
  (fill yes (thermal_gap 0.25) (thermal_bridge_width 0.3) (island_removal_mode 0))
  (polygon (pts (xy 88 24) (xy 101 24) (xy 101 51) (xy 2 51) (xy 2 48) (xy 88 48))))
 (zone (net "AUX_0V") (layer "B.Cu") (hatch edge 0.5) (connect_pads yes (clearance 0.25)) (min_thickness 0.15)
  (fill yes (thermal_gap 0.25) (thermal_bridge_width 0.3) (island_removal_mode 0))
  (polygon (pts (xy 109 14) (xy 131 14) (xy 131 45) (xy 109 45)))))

